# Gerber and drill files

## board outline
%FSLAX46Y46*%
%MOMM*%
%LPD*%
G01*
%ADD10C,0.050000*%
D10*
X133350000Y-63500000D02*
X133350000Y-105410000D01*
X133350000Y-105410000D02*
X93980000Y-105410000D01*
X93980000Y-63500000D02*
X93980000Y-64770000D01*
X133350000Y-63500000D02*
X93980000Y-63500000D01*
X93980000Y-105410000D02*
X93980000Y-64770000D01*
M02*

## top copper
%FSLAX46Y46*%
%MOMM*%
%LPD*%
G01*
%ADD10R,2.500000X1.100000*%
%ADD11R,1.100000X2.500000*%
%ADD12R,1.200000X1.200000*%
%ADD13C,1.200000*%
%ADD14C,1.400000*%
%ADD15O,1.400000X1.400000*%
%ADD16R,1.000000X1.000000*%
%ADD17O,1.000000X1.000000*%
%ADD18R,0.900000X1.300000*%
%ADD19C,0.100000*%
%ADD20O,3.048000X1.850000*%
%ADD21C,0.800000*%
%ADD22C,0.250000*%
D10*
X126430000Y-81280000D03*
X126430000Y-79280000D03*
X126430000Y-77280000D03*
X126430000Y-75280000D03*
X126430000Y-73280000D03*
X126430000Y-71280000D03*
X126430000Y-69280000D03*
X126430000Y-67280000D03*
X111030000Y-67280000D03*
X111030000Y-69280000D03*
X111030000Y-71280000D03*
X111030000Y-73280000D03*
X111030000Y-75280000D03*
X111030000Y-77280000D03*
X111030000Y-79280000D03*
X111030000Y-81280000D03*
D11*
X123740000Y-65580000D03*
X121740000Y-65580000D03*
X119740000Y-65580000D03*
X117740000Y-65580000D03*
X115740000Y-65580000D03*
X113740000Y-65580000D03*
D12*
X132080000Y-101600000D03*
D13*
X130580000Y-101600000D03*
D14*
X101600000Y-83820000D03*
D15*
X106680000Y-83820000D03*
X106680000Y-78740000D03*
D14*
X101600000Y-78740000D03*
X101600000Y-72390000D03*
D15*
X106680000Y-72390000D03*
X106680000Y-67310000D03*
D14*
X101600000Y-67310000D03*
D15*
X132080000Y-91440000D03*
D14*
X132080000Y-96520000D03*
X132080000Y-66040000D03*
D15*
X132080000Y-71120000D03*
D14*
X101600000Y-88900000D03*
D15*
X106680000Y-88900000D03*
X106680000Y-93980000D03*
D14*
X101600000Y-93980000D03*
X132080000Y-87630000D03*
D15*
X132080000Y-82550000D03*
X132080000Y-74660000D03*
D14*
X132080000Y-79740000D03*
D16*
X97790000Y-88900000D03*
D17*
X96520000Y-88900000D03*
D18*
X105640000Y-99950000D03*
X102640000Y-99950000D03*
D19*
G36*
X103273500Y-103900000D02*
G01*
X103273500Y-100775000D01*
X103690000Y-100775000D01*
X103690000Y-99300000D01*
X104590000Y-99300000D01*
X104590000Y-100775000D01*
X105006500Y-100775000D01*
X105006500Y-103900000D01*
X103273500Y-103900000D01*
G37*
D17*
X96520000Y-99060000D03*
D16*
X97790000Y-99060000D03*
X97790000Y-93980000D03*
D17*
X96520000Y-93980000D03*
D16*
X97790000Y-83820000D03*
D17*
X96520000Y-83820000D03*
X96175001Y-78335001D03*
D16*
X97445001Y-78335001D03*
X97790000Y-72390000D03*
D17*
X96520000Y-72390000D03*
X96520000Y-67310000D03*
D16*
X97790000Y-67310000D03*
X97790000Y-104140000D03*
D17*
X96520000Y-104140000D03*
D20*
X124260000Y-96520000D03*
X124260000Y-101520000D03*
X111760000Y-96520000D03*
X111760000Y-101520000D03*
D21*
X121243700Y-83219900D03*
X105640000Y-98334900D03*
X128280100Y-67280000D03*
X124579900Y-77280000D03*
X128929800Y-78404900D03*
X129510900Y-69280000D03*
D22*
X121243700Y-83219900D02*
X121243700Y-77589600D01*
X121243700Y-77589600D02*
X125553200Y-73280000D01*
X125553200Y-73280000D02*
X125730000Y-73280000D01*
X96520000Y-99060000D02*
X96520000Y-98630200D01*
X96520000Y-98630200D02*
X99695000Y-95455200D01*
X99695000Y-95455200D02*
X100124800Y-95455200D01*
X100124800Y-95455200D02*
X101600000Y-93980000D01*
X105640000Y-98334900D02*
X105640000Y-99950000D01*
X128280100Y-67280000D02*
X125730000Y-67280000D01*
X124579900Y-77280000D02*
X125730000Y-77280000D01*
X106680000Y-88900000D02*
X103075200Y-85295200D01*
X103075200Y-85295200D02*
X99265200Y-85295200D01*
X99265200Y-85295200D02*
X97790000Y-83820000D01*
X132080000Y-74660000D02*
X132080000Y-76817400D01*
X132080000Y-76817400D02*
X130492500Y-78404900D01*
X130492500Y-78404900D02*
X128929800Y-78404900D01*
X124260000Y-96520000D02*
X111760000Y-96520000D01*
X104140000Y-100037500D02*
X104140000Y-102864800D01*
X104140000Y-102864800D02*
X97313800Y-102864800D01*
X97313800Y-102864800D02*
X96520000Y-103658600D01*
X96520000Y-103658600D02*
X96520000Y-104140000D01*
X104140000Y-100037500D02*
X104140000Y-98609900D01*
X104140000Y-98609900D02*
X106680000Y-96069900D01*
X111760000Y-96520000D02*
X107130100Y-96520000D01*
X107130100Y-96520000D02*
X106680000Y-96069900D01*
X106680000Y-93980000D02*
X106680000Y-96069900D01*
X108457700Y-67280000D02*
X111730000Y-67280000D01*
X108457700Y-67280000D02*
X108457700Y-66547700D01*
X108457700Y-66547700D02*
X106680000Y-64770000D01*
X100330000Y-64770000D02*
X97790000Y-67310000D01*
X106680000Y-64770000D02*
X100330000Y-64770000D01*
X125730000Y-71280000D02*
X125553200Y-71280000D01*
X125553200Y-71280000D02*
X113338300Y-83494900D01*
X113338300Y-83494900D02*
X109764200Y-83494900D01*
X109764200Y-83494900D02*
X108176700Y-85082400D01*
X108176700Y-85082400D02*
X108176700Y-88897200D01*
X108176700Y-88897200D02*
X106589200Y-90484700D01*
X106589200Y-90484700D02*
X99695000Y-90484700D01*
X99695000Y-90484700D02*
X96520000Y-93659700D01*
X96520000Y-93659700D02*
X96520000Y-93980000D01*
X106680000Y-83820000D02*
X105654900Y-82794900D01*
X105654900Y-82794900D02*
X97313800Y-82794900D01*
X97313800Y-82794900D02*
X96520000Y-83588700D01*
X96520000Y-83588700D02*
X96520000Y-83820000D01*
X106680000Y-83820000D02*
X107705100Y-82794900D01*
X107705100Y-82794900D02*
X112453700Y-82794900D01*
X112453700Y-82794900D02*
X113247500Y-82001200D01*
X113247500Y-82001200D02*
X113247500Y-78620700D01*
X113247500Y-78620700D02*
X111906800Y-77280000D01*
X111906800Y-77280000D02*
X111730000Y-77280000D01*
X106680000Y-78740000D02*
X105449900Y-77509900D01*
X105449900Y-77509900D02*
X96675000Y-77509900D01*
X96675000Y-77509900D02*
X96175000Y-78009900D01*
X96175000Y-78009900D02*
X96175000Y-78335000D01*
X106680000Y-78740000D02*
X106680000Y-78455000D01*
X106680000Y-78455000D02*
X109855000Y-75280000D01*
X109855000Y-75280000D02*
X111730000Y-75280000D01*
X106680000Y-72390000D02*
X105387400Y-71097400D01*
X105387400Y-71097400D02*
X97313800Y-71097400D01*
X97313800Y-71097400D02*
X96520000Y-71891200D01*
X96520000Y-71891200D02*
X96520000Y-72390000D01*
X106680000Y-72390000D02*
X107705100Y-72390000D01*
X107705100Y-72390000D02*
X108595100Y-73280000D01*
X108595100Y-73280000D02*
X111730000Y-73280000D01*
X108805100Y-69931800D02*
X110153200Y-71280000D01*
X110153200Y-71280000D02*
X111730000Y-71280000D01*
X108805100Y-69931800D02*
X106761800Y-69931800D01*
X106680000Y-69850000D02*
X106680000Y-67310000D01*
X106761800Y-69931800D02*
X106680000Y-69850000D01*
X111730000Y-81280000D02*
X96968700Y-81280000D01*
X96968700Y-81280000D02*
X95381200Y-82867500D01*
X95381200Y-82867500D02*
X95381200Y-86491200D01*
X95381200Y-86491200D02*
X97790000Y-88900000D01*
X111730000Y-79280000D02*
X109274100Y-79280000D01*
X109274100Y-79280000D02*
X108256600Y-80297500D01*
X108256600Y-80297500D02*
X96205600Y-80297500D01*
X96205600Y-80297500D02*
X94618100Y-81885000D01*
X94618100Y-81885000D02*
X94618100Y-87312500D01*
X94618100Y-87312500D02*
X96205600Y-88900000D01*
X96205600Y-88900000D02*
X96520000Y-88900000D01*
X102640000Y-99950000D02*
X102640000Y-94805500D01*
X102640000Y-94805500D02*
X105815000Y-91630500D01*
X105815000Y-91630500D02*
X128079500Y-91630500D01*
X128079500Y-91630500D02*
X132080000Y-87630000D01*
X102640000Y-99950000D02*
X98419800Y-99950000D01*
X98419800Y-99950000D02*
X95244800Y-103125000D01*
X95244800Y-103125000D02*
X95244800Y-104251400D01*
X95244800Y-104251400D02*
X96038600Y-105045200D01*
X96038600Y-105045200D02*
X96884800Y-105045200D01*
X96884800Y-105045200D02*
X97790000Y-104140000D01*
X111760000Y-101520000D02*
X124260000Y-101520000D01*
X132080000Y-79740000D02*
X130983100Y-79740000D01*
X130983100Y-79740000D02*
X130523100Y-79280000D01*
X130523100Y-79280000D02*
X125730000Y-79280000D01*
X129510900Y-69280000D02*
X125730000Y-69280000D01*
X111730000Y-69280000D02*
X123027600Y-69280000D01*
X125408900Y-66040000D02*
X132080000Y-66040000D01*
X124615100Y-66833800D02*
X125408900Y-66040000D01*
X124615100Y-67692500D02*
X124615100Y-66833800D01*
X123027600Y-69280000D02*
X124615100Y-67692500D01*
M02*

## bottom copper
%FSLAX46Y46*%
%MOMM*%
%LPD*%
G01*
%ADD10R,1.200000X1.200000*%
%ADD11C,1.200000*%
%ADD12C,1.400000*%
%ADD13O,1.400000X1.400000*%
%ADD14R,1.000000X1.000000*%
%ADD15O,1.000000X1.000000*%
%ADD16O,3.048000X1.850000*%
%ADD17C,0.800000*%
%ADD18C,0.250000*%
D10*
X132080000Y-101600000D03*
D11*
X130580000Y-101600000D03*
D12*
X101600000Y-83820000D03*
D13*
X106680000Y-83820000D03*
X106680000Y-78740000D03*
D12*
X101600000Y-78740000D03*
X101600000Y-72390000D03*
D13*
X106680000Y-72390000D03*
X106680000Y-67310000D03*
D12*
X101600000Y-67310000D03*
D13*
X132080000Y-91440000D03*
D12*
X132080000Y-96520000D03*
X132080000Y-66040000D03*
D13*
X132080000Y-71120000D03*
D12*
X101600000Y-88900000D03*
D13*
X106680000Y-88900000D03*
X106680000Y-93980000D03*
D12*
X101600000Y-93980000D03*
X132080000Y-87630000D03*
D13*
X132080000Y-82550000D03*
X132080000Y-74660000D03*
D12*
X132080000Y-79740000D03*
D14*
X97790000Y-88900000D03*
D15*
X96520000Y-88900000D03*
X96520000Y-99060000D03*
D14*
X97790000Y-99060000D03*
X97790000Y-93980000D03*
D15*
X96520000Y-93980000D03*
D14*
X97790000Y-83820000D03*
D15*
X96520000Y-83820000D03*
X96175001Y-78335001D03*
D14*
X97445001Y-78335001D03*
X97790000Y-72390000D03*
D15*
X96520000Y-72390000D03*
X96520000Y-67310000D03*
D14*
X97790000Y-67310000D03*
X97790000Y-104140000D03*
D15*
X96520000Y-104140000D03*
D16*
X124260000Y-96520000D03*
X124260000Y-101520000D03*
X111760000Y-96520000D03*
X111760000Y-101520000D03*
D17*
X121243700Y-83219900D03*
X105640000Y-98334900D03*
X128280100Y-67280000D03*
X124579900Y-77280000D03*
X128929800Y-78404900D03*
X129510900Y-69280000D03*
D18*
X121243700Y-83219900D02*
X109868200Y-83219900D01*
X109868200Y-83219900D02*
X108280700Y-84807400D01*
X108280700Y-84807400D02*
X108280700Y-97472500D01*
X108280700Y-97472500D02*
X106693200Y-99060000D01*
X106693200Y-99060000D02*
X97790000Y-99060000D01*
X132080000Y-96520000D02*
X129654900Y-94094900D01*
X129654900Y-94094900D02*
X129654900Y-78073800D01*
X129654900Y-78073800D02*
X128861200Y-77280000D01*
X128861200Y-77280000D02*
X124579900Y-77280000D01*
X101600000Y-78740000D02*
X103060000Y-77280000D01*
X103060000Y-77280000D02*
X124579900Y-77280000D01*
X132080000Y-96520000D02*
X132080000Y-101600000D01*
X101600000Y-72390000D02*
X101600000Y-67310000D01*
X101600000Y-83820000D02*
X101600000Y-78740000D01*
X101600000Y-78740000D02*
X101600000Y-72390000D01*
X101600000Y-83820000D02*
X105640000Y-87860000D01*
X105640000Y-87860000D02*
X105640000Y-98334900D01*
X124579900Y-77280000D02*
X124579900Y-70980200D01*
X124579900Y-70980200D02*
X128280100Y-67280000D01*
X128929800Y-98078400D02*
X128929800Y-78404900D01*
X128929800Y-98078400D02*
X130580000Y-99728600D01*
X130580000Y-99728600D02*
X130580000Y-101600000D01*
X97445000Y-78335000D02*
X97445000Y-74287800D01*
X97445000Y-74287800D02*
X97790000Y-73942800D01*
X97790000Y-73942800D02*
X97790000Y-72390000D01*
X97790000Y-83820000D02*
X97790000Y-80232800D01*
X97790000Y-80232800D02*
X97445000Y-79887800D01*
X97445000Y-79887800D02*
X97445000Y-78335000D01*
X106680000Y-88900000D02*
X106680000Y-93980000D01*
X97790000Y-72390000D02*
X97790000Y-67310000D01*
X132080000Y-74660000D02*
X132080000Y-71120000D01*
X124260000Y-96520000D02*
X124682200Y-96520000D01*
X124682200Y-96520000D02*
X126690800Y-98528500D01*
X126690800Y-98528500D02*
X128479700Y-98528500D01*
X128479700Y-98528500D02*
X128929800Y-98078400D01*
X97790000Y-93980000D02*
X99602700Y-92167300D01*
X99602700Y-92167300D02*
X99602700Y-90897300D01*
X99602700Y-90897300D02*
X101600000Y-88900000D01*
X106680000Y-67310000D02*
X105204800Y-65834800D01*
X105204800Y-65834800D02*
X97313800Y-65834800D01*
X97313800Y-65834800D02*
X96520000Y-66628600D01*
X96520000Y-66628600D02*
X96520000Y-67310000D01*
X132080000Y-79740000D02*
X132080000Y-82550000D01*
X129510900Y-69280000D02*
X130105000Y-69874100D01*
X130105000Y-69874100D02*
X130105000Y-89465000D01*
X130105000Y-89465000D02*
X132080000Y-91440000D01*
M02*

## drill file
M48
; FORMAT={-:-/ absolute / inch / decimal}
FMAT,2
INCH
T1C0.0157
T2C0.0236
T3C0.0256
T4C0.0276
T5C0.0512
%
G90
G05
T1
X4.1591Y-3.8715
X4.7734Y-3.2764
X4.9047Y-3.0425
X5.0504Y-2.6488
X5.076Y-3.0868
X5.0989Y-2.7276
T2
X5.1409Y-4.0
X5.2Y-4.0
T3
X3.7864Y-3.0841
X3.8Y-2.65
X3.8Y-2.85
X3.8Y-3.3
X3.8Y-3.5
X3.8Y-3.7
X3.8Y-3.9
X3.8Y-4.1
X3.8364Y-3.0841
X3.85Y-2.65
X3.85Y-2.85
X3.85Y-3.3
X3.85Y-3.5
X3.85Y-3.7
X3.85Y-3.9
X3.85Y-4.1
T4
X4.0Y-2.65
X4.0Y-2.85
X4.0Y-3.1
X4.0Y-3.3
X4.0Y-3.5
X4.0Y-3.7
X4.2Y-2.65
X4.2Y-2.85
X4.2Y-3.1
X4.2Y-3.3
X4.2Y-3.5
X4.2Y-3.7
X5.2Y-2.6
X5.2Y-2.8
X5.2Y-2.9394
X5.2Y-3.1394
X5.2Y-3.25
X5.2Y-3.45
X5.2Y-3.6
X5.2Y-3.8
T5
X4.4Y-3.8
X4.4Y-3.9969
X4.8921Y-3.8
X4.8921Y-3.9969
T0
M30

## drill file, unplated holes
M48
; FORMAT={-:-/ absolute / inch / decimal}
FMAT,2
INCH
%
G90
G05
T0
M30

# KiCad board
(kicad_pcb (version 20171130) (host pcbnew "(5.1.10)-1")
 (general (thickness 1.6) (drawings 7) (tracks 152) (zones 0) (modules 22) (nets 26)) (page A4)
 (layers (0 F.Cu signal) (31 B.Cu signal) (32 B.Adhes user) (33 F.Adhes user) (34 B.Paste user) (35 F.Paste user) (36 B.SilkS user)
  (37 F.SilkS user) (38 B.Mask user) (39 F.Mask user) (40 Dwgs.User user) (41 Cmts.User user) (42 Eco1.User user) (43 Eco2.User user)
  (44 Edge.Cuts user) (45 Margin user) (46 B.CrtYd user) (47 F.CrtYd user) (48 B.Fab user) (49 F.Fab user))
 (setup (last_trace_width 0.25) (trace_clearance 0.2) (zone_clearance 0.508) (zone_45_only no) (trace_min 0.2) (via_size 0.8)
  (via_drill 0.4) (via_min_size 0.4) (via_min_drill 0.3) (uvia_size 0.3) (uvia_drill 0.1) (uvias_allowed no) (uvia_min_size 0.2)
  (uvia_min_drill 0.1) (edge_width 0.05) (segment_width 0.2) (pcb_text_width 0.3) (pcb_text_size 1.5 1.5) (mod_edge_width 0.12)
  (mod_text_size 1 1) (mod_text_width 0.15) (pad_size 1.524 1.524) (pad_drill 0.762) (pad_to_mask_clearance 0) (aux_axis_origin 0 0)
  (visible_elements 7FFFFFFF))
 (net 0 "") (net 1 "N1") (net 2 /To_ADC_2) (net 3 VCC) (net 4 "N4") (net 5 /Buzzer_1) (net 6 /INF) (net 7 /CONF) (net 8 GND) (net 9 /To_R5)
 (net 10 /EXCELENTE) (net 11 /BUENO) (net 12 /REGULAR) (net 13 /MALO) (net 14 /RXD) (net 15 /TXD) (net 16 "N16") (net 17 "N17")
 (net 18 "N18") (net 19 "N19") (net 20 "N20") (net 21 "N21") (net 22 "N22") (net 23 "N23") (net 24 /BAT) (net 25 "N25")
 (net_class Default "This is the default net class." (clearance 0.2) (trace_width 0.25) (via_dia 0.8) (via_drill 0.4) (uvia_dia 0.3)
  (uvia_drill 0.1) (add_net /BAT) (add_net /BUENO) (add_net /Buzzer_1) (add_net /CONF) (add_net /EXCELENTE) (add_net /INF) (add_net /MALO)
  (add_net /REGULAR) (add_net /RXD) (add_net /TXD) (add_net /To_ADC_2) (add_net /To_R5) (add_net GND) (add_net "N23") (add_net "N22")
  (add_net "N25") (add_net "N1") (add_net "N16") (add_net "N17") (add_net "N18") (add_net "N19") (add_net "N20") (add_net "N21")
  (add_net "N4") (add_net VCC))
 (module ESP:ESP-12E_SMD (layer F.Cu) (at 125.73 81.28 180)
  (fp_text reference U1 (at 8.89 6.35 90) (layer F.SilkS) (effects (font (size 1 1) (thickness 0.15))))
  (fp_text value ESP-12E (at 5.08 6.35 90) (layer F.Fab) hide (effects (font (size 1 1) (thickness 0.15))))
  (pad 1 smd rect (at 0 0 180) (size 2.5 1.1) (drill (offset -0.7 0)) (layers F.Cu F.Paste F.Mask) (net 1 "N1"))
  (pad 2 smd rect (at 0 2 180) (size 2.5 1.1) (drill (offset -0.7 0)) (layers F.Cu F.Paste F.Mask) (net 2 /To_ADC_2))
  (pad 3 smd rect (at 0 4 180) (size 2.5 1.1) (drill (offset -0.7 0)) (layers F.Cu F.Paste F.Mask) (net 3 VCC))
  (pad 4 smd rect (at 0 6 180) (size 2.5 1.1) (drill (offset -0.7 0)) (layers F.Cu F.Paste F.Mask) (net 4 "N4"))
  (pad 5 smd rect (at 0 8 180) (size 2.5 1.1) (drill (offset -0.7 0)) (layers F.Cu F.Paste F.Mask) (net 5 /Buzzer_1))
  (pad 6 smd rect (at 0 10 180) (size 2.5 1.1) (drill (offset -0.7 0)) (layers F.Cu F.Paste F.Mask) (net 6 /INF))
  (pad 7 smd rect (at 0 12 180) (size 2.5 1.1) (drill (offset -0.7 0)) (layers F.Cu F.Paste F.Mask) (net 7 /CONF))
  (pad 8 smd rect (at 0 14 180) (size 2.5 1.1) (drill (offset -0.7 0)) (layers F.Cu F.Paste F.Mask) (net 3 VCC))
  (pad 9 smd rect (at 14 14 180) (size 2.5 1.1) (drill (offset 0.7 0)) (layers F.Cu F.Paste F.Mask) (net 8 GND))
  (pad 10 smd rect (at 14 12 180) (size 2.5 1.1) (drill (offset 0.7 0)) (layers F.Cu F.Paste F.Mask) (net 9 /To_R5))
  (pad 11 smd rect (at 14 10 180) (size 2.5 1.1) (drill (offset 0.7 0)) (layers F.Cu F.Paste F.Mask) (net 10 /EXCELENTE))
  (pad 12 smd rect (at 14 8 180) (size 2.5 1.1) (drill (offset 0.7 0)) (layers F.Cu F.Paste F.Mask) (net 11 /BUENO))
  (pad 13 smd rect (at 14 6 180) (size 2.5 1.1) (drill (offset 0.7 0)) (layers F.Cu F.Paste F.Mask) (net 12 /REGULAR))
  (pad 14 smd rect (at 14 4 180) (size 2.5 1.1) (drill (offset 0.7 0)) (layers F.Cu F.Paste F.Mask) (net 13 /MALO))
  (pad 15 smd rect (at 14 2 180) (size 2.5 1.1) (drill (offset 0.7 0)) (layers F.Cu F.Paste F.Mask) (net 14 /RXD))
  (pad 16 smd rect (at 14 0 180) (size 2.5 1.1) (drill (offset 0.7 0)) (layers F.Cu F.Paste F.Mask) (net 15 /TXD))
  (pad 17 smd rect (at 1.99 15 270) (size 2.5 1.1) (drill (offset -0.7 0)) (layers F.Cu F.Paste F.Mask) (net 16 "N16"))
  (pad 18 smd rect (at 3.99 15 270) (size 2.5 1.1) (drill (offset -0.7 0)) (layers F.Cu F.Paste F.Mask) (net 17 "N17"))
  (pad 19 smd rect (at 5.99 15 270) (size 2.5 1.1) (drill (offset -0.7 0)) (layers F.Cu F.Paste F.Mask) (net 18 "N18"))
  (pad 20 smd rect (at 7.99 15 270) (size 2.5 1.1) (drill (offset -0.7 0)) (layers F.Cu F.Paste F.Mask) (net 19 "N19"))
  (pad 21 smd rect (at 9.99 15 270) (size 2.5 1.1) (drill (offset -0.7 0)) (layers F.Cu F.Paste F.Mask) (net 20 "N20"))
  (pad 22 smd rect (at 11.99 15 270) (size 2.5 1.1) (drill (offset -0.7 0)) (layers F.Cu F.Paste F.Mask) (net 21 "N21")))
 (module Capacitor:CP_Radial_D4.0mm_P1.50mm (layer F.Cu) (at 132.08 101.6 180)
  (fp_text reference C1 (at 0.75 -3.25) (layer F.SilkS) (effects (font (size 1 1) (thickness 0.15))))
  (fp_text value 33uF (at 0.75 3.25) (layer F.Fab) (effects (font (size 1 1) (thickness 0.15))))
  (pad 1 thru_hole rect (at 0 0 180) (size 1.2 1.2) (drill 0.6) (layers *.Cu *.Mask) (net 3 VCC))
  (pad 2 thru_hole circle (at 1.5 0 180) (size 1.2 1.2) (drill 0.6) (layers *.Cu *.Mask) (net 8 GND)))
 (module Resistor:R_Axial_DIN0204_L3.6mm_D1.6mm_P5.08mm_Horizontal (layer F.Cu) (at 101.6 83.82)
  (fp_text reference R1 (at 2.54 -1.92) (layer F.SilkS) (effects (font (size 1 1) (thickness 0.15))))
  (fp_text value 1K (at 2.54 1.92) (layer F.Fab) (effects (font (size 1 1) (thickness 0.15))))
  (pad 1 thru_hole circle (at 0 0) (size 1.4 1.4) (drill 0.7) (layers *.Cu *.Mask) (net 3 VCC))
  (pad 2 thru_hole oval (at 5.08 0) (size 1.4 1.4) (drill 0.7) (layers *.Cu *.Mask) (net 13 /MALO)))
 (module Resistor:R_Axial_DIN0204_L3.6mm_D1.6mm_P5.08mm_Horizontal (layer F.Cu) (at 101.6 78.74)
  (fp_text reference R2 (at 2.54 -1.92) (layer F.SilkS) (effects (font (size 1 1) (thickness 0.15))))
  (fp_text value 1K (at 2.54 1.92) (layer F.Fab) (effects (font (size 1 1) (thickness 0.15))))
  (pad 2 thru_hole oval (at 5.08 0) (size 1.4 1.4) (drill 0.7) (layers *.Cu *.Mask) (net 12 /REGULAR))
  (pad 1 thru_hole circle (at 0 0) (size 1.4 1.4) (drill 0.7) (layers *.Cu *.Mask) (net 3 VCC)))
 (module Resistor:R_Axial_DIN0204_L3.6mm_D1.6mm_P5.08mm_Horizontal (layer F.Cu) (at 101.6 72.39)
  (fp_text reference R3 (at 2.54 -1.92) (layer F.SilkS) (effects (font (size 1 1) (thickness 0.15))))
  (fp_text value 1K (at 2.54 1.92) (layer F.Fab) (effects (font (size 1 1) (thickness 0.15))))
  (pad 1 thru_hole circle (at 0 0) (size 1.4 1.4) (drill 0.7) (layers *.Cu *.Mask) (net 3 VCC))
  (pad 2 thru_hole oval (at 5.08 0) (size 1.4 1.4) (drill 0.7) (layers *.Cu *.Mask) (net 11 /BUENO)))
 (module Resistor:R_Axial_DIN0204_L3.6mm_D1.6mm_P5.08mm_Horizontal (layer F.Cu) (at 101.6 67.31)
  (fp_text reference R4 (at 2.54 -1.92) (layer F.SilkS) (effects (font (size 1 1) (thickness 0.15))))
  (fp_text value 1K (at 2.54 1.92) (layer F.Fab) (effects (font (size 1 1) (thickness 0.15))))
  (pad 2 thru_hole oval (at 5.08 0) (size 1.4 1.4) (drill 0.7) (layers *.Cu *.Mask) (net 10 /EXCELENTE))
  (pad 1 thru_hole circle (at 0 0) (size 1.4 1.4) (drill 0.7) (layers *.Cu *.Mask) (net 3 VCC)))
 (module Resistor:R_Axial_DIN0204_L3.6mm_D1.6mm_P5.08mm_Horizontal (layer F.Cu) (at 132.08 96.52 90)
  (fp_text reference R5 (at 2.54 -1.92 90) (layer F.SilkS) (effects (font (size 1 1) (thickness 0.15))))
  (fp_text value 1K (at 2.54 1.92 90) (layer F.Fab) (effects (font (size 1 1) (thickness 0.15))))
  (pad 2 thru_hole oval (at 5.08 0 90) (size 1.4 1.4) (drill 0.7) (layers *.Cu *.Mask) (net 7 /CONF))
  (pad 1 thru_hole circle (at 0 0 90) (size 1.4 1.4) (drill 0.7) (layers *.Cu *.Mask) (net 3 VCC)))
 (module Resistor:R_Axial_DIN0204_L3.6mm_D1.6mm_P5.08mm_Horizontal (layer F.Cu) (at 132.08 66.04 270)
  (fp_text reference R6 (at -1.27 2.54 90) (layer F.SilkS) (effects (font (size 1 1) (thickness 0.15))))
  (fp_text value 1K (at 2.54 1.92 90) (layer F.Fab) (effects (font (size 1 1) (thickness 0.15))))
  (pad 1 thru_hole circle (at 0 0 270) (size 1.4 1.4) (drill 0.7) (layers *.Cu *.Mask) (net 9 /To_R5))
  (pad 2 thru_hole oval (at 5.08 0 270) (size 1.4 1.4) (drill 0.7) (layers *.Cu *.Mask) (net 8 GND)))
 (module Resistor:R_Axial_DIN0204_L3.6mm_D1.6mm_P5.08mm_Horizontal (layer F.Cu) (at 101.6 88.9)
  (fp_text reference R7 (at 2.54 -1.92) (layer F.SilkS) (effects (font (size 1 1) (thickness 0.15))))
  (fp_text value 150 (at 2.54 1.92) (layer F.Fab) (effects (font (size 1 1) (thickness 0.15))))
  (pad 1 thru_hole circle (at 0 0) (size 1.4 1.4) (drill 0.7) (layers *.Cu *.Mask) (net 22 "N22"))
  (pad 2 thru_hole oval (at 5.08 0) (size 1.4 1.4) (drill 0.7) (layers *.Cu *.Mask) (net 8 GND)))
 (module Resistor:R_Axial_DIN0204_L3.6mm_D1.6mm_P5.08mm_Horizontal (layer F.Cu) (at 101.6 93.98)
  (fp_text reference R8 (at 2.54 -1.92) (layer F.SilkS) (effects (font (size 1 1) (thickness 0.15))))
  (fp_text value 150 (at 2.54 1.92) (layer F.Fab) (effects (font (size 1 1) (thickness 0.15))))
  (pad 2 thru_hole oval (at 5.08 0) (size 1.4 1.4) (drill 0.7) (layers *.Cu *.Mask) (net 8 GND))
  (pad 1 thru_hole circle (at 0 0) (size 1.4 1.4) (drill 0.7) (layers *.Cu *.Mask) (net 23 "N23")))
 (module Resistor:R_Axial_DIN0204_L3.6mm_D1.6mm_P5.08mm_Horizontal (layer F.Cu) (at 132.08 87.63 90)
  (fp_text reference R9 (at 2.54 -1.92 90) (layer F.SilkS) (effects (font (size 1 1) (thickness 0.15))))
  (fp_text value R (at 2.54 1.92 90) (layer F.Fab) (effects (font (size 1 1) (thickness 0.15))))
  (pad 1 thru_hole circle (at 0 0 90) (size 1.4 1.4) (drill 0.7) (layers *.Cu *.Mask) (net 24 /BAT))
  (pad 2 thru_hole oval (at 5.08 0 90) (size 1.4 1.4) (drill 0.7) (layers *.Cu *.Mask) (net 2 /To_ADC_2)))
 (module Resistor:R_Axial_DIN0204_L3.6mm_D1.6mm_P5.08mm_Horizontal (layer F.Cu) (at 132.08 79.74 90)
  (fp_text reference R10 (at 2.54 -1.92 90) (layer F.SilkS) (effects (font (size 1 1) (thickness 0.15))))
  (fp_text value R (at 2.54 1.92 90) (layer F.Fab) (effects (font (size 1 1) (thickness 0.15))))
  (pad 2 thru_hole oval (at 5.08 0 90) (size 1.4 1.4) (drill 0.7) (layers *.Cu *.Mask) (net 8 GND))
  (pad 1 thru_hole circle (at 0 0 90) (size 1.4 1.4) (drill 0.7) (layers *.Cu *.Mask) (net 2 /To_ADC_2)))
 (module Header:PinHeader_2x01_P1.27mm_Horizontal (layer F.Cu) (at 97.79 88.9 180)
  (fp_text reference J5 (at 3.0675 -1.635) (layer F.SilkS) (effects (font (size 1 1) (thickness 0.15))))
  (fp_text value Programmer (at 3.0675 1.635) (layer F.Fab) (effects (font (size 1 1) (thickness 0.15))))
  (pad 1 thru_hole rect (at 0 0 180) (size 1 1) (drill 0.65) (layers *.Cu *.Mask) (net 15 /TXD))
  (pad 2 thru_hole oval (at 1.27 0 180) (size 1 1) (drill 0.65) (layers *.Cu *.Mask) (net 14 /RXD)))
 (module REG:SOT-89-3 (layer F.Cu) (at 104.14 101.6 270)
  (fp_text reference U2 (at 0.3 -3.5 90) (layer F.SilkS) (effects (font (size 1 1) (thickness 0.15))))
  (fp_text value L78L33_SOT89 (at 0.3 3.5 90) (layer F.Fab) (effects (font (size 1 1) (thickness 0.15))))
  (pad 1 smd rect (at -1.65 -1.5 270) (size 1.3 0.9) (layers F.Cu F.Paste F.Mask) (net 3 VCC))
  (pad 3 smd rect (at -1.65 1.5 270) (size 1.3 0.9) (layers F.Cu F.Paste F.Mask) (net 24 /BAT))
  (pad 2 smd custom (at -1.5625 0 270) (size 1.475 0.9) (layers F.Cu F.Paste F.Mask) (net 8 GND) (zone_connect 2)
   (options (clearance outline) (anchor rect)) (primitives)))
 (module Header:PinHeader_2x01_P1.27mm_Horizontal (layer F.Cu) (at 97.79 99.06 180)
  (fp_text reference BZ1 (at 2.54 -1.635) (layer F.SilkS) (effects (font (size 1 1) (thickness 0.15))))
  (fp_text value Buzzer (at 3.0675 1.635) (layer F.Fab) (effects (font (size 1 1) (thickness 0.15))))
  (pad 2 thru_hole oval (at 1.27 0 180) (size 1 1) (drill 0.65) (layers *.Cu *.Mask) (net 23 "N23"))
  (pad 1 thru_hole rect (at 0 0 180) (size 1 1) (drill 0.65) (layers *.Cu *.Mask) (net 5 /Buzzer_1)))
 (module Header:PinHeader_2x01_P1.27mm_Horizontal (layer F.Cu) (at 97.79 93.98 180)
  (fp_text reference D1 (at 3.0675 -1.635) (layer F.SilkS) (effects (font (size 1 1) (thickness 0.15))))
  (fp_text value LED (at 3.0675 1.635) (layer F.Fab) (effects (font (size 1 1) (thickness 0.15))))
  (pad 1 thru_hole rect (at 0 0 180) (size 1 1) (drill 0.65) (layers *.Cu *.Mask) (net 22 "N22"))
  (pad 2 thru_hole oval (at 1.27 0 180) (size 1 1) (drill 0.65) (layers *.Cu *.Mask) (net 6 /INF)))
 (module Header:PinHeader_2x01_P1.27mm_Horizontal (layer F.Cu) (at 97.79 83.82 180)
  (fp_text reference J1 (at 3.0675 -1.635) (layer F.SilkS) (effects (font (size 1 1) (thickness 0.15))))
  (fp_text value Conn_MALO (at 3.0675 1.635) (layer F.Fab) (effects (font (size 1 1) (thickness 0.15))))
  (pad 1 thru_hole rect (at 0 0 180) (size 1 1) (drill 0.65) (layers *.Cu *.Mask) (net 8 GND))
  (pad 2 thru_hole oval (at 1.27 0 180) (size 1 1) (drill 0.65) (layers *.Cu *.Mask) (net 13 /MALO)))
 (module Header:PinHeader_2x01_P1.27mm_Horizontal (layer F.Cu) (at 97.445001 78.335001 180)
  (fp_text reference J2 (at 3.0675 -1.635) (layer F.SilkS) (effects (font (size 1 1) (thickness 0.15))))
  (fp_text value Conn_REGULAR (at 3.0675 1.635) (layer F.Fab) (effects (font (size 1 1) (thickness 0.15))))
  (pad 2 thru_hole oval (at 1.27 0 180) (size 1 1) (drill 0.65) (layers *.Cu *.Mask) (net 12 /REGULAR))
  (pad 1 thru_hole rect (at 0 0 180) (size 1 1) (drill 0.65) (layers *.Cu *.Mask) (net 8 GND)))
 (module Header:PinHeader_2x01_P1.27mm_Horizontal (layer F.Cu) (at 97.79 72.39 180)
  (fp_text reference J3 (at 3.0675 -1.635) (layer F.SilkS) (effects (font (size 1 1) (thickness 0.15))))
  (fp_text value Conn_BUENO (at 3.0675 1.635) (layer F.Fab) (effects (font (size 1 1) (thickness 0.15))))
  (pad 1 thru_hole rect (at 0 0 180) (size 1 1) (drill 0.65) (layers *.Cu *.Mask) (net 8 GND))
  (pad 2 thru_hole oval (at 1.27 0 180) (size 1 1) (drill 0.65) (layers *.Cu *.Mask) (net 11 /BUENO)))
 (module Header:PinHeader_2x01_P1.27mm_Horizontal (layer F.Cu) (at 97.79 67.31 180)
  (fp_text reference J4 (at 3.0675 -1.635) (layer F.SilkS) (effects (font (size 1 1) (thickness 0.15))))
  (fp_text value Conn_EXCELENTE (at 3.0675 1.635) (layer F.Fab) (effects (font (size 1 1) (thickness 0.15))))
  (pad 2 thru_hole oval (at 1.27 0 180) (size 1 1) (drill 0.65) (layers *.Cu *.Mask) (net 10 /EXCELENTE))
  (pad 1 thru_hole rect (at 0 0 180) (size 1 1) (drill 0.65) (layers *.Cu *.Mask) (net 8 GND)))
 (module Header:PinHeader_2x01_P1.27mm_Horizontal (layer F.Cu) (at 97.79 104.14 180)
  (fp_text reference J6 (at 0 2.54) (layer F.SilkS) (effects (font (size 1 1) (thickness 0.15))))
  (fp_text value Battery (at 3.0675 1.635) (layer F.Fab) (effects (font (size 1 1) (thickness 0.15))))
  (pad 1 thru_hole rect (at 0 0 180) (size 1 1) (drill 0.65) (layers *.Cu *.Mask) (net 24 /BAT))
  (pad 2 thru_hole oval (at 1.27 0 180) (size 1 1) (drill 0.65) (layers *.Cu *.Mask) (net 8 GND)))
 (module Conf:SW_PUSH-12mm (layer F.Cu) (at 111.76 96.52)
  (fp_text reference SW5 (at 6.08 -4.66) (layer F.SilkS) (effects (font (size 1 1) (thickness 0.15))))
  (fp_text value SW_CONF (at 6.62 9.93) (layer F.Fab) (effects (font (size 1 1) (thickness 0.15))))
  (pad 1 thru_hole oval (at 12.5 0) (size 3.048 1.85) (drill 1.3) (layers *.Cu *.Mask) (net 8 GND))
  (pad 2 thru_hole oval (at 12.5 5) (size 3.048 1.85) (drill 1.3) (layers *.Cu *.Mask) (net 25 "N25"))
  (pad 1 thru_hole oval (at 0 0) (size 3.048 1.85) (drill 1.3) (layers *.Cu *.Mask) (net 8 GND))
  (pad 2 thru_hole oval (at 0 5) (size 3.048 1.85) (drill 1.3) (layers *.Cu *.Mask) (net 25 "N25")))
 (gr_line (start 133.35 63.5) (end 133.35 105.41) (layer Edge.Cuts) (width 0.05))
 (gr_line (start 133.35 105.41) (end 93.98 105.41) (layer Edge.Cuts) (width 0.05))
 (gr_line (start 93.98 63.5) (end 93.98 64.77) (layer Edge.Cuts) (width 0.05))
 (gr_line (start 133.35 63.5) (end 93.98 63.5) (layer Edge.Cuts) (width 0.05))
 (gr_line (start 93.98 105.41) (end 93.98 64.77) (layer Edge.Cuts) (width 0.05))
 (segment (start 121.2437 83.2199) (end 121.2437 77.5896) (width 0.25) (layer F.Cu) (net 5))
 (segment (start 121.2437 77.5896) (end 125.5532 73.28) (width 0.25) (layer F.Cu) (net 5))
 (segment (start 125.5532 73.28) (end 125.73 73.28) (width 0.25) (layer F.Cu) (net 5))
 (segment (start 121.2437 83.2199) (end 109.8682 83.2199) (width 0.25) (layer B.Cu) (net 5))
 (segment (start 109.8682 83.2199) (end 108.2807 84.8074) (width 0.25) (layer B.Cu) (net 5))
 (segment (start 108.2807 84.8074) (end 108.2807 97.4725) (width 0.25) (layer B.Cu) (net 5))
 (segment (start 108.2807 97.4725) (end 106.6932 99.06) (width 0.25) (layer B.Cu) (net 5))
 (segment (start 106.6932 99.06) (end 97.79 99.06) (width 0.25) (layer B.Cu) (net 5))
 (via (at 121.2437 83.2199) (size 0.8) (layers F.Cu B.Cu) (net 5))
 (segment (start 96.52 99.06) (end 96.52 98.6302) (width 0.25) (layer F.Cu) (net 23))
 (segment (start 96.52 98.6302) (end 99.695 95.4552) (width 0.25) (layer F.Cu) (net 23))
 (segment (start 99.695 95.4552) (end 100.1248 95.4552) (width 0.25) (layer F.Cu) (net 23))
 (segment (start 100.1248 95.4552) (end 101.6 93.98) (width 0.25) (layer F.Cu) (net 23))
 (segment (start 132.08 96.52) (end 129.6549 94.0949) (width 0.25) (layer B.Cu) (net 3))
 (segment (start 129.6549 94.0949) (end 129.6549 78.0738) (width 0.25) (layer B.Cu) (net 3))
 (segment (start 129.6549 78.0738) (end 128.8612 77.28) (width 0.25) (layer B.Cu) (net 3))
 (segment (start 128.8612 77.28) (end 124.5799 77.28) (width 0.25) (layer B.Cu) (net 3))
 (segment (start 101.6 78.74) (end 103.06 77.28) (width 0.25) (layer B.Cu) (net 3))
 (segment (start 103.06 77.28) (end 124.5799 77.28) (width 0.25) (layer B.Cu) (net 3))
 (segment (start 132.08 96.52) (end 132.08 101.6) (width 0.25) (layer B.Cu) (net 3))
 (segment (start 101.6 72.39) (end 101.6 67.31) (width 0.25) (layer B.Cu) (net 3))
 (segment (start 101.6 83.82) (end 101.6 78.74) (width 0.25) (layer B.Cu) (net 3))
 (segment (start 101.6 78.74) (end 101.6 72.39) (width 0.25) (layer B.Cu) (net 3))
 (segment (start 105.64 98.3349) (end 105.64 99.95) (width 0.25) (layer F.Cu) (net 3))
 (segment (start 101.6 83.82) (end 105.64 87.86) (width 0.25) (layer B.Cu) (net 3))
 (segment (start 105.64 87.86) (end 105.64 98.3349) (width 0.25) (layer B.Cu) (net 3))
 (segment (start 128.2801 67.28) (end 125.73 67.28) (width 0.25) (layer F.Cu) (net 3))
 (segment (start 124.5799 77.28) (end 124.5799 70.9802) (width 0.25) (layer B.Cu) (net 3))
 (segment (start 124.5799 70.9802) (end 128.2801 67.28) (width 0.25) (layer B.Cu) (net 3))
 (segment (start 124.5799 77.28) (end 125.73 77.28) (width 0.25) (layer F.Cu) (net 3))
 (via (at 105.64 98.3349) (size 0.8) (layers F.Cu B.Cu) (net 3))
 (via (at 128.2801 67.28) (size 0.8) (layers F.Cu B.Cu) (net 3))
 (via (at 124.5799 77.28) (size 0.8) (layers F.Cu B.Cu) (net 3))
 (segment (start 106.68 88.9) (end 103.0752 85.2952) (width 0.25) (layer F.Cu) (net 8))
 (segment (start 103.0752 85.2952) (end 99.2652 85.2952) (width 0.25) (layer F.Cu) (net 8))
 (segment (start 99.2652 85.2952) (end 97.79 83.82) (width 0.25) (layer F.Cu) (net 8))
 (segment (start 132.08 74.66) (end 132.08 76.8174) (width 0.25) (layer F.Cu) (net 8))
 (segment (start 132.08 76.8174) (end 130.4925 78.4049) (width 0.25) (layer F.Cu) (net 8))
 (segment (start 130.4925 78.4049) (end 128.9298 78.4049) (width 0.25) (layer F.Cu) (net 8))
 (segment (start 128.9298 98.0784) (end 128.9298 78.4049) (width 0.25) (layer B.Cu) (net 8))
 (segment (start 128.9298 98.0784) (end 130.58 99.7286) (width 0.25) (layer B.Cu) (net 8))
 (segment (start 130.58 99.7286) (end 130.58 101.6) (width 0.25) (layer B.Cu) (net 8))
 (segment (start 124.26 96.52) (end 111.76 96.52) (width 0.25) (layer F.Cu) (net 8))
 (segment (start 104.14 100.0375) (end 104.14 102.8648) (width 0.25) (layer F.Cu) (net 8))
 (segment (start 104.14 102.8648) (end 97.3138 102.8648) (width 0.25) (layer F.Cu) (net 8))
 (segment (start 97.3138 102.8648) (end 96.52 103.6586) (width 0.25) (layer F.Cu) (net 8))
 (segment (start 96.52 103.6586) (end 96.52 104.14) (width 0.25) (layer F.Cu) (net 8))
 (segment (start 97.445 78.335) (end 97.445 74.2878) (width 0.25) (layer B.Cu) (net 8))
 (segment (start 97.445 74.2878) (end 97.79 73.9428) (width 0.25) (layer B.Cu) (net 8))
 (segment (start 97.79 73.9428) (end 97.79 72.39) (width 0.25) (layer B.Cu) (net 8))
 (segment (start 104.14 100.0375) (end 104.14 98.6099) (width 0.25) (layer F.Cu) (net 8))
 (segment (start 104.14 98.6099) (end 106.68 96.0699) (width 0.25) (layer F.Cu) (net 8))
 (segment (start 97.79 83.82) (end 97.79 80.2328) (width 0.25) (layer B.Cu) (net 8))
 (segment (start 97.79 80.2328) (end 97.445 79.8878) (width 0.25) (layer B.Cu) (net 8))
 (segment (start 97.445 79.8878) (end 97.445 78.335) (width 0.25) (layer B.Cu) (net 8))
 (segment (start 111.76 96.52) (end 107.1301 96.52) (width 0.25) (layer F.Cu) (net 8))
 (segment (start 107.1301 96.52) (end 106.68 96.0699) (width 0.25) (layer F.Cu) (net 8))
 (segment (start 106.68 88.9) (end 106.68 93.98) (width 0.25) (layer B.Cu) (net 8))
 (segment (start 97.79 72.39) (end 97.79 67.31) (width 0.25) (layer B.Cu) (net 8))
 (segment (start 132.08 74.66) (end 132.08 71.12) (width 0.25) (layer B.Cu) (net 8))
 (segment (start 124.26 96.52) (end 124.6822 96.52) (width 0.25) (layer B.Cu) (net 8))
 (segment (start 124.6822 96.52) (end 126.6908 98.5285) (width 0.25) (layer B.Cu) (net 8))
 (segment (start 126.6908 98.5285) (end 128.4797 98.5285) (width 0.25) (layer B.Cu) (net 8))
 (segment (start 128.4797 98.5285) (end 128.9298 98.0784) (width 0.25) (layer B.Cu) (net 8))
 (segment (start 106.68 93.98) (end 106.68 96.0699) (width 0.25) (layer F.Cu) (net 8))
 (segment (start 108.4577 67.28) (end 111.73 67.28) (width 0.25) (layer F.Cu) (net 8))
 (via (at 128.9298 78.4049) (size 0.8) (layers F.Cu B.Cu) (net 8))
 (segment (start 108.4577 67.28) (end 108.4577 66.5477) (width 0.25) (layer F.Cu) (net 8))
 (segment (start 108.4577 66.5477) (end 106.68 64.77) (width 0.25) (layer F.Cu) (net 8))
 (segment (start 100.33 64.77) (end 97.79 67.31) (width 0.25) (layer F.Cu) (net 8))
 (segment (start 106.68 64.77) (end 100.33 64.77) (width 0.25) (layer F.Cu) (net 8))
 (segment (start 97.79 93.98) (end 99.6027 92.1673) (width 0.25) (layer B.Cu) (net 22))
 (segment (start 99.6027 92.1673) (end 99.6027 90.8973) (width 0.25) (layer B.Cu) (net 22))
 (segment (start 99.6027 90.8973) (end 101.6 88.9) (width 0.25) (layer B.Cu) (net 22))
 (segment (start 125.73 71.28) (end 125.5532 71.28) (width 0.25) (layer F.Cu) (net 6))
 (segment (start 125.5532 71.28) (end 113.3383 83.4949) (width 0.25) (layer F.Cu) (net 6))
 (segment (start 113.3383 83.4949) (end 109.7642 83.4949) (width 0.25) (layer F.Cu) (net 6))
 (segment (start 109.7642 83.4949) (end 108.1767 85.0824) (width 0.25) (layer F.Cu) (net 6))
 (segment (start 108.1767 85.0824) (end 108.1767 88.8972) (width 0.25) (layer F.Cu) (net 6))
 (segment (start 108.1767 88.8972) (end 106.5892 90.4847) (width 0.25) (layer F.Cu) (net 6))
 (segment (start 106.5892 90.4847) (end 99.695 90.4847) (width 0.25) (layer F.Cu) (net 6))
 (segment (start 99.695 90.4847) (end 96.52 93.6597) (width 0.25) (layer F.Cu) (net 6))
 (segment (start 96.52 93.6597) (end 96.52 93.98) (width 0.25) (layer F.Cu) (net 6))
 (segment (start 106.68 83.82) (end 105.6549 82.7949) (width 0.25) (layer F.Cu) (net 13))
 (segment (start 105.6549 82.7949) (end 97.3138 82.7949) (width 0.25) (layer F.Cu) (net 13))
 (segment (start 97.3138 82.7949) (end 96.52 83.5887) (width 0.25) (layer F.Cu) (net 13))
 (segment (start 96.52 83.5887) (end 96.52 83.82) (width 0.25) (layer F.Cu) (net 13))
 (segment (start 106.68 83.82) (end 107.7051 82.7949) (width 0.25) (layer F.Cu) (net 13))
 (segment (start 107.7051 82.7949) (end 112.4537 82.7949) (width 0.25) (layer F.Cu) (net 13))
 (segment (start 112.4537 82.7949) (end 113.2475 82.0012) (width 0.25) (layer F.Cu) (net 13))
 (segment (start 113.2475 82.0012) (end 113.2475 78.6207) (width 0.25) (layer F.Cu) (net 13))
 (segment (start 113.2475 78.6207) (end 111.9068 77.28) (width 0.25) (layer F.Cu) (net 13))
 (segment (start 111.9068 77.28) (end 111.73 77.28) (width 0.25) (layer F.Cu) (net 13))
 (segment (start 106.68 78.74) (end 105.4499 77.5099) (width 0.25) (layer F.Cu) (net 12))
 (segment (start 105.4499 77.5099) (end 96.675 77.5099) (width 0.25) (layer F.Cu) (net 12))
 (segment (start 96.675 77.5099) (end 96.175 78.0099) (width 0.25) (layer F.Cu) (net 12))
 (segment (start 96.175 78.0099) (end 96.175 78.335) (width 0.25) (layer F.Cu) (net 12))
 (segment (start 106.68 78.74) (end 106.68 78.455) (width 0.25) (layer F.Cu) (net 12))
 (segment (start 106.68 78.455) (end 109.855 75.28) (width 0.25) (layer F.Cu) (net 12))
 (segment (start 109.855 75.28) (end 111.73 75.28) (width 0.25) (layer F.Cu) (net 12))
 (segment (start 106.68 72.39) (end 105.3874 71.0974) (width 0.25) (layer F.Cu) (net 11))
 (segment (start 105.3874 71.0974) (end 97.3138 71.0974) (width 0.25) (layer F.Cu) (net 11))
 (segment (start 97.3138 71.0974) (end 96.52 71.8912) (width 0.25) (layer F.Cu) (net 11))
 (segment (start 96.52 71.8912) (end 96.52 72.39) (width 0.25) (layer F.Cu) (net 11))
 (segment (start 106.68 72.39) (end 107.7051 72.39) (width 0.25) (layer F.Cu) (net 11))
 (segment (start 107.7051 72.39) (end 108.5951 73.28) (width 0.25) (layer F.Cu) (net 11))
 (segment (start 108.5951 73.28) (end 111.73 73.28) (width 0.25) (layer F.Cu) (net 11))
 (segment (start 106.68 67.31) (end 105.2048 65.8348) (width 0.25) (layer B.Cu) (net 10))
 (segment (start 105.2048 65.8348) (end 97.3138 65.8348) (width 0.25) (layer B.Cu) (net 10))
 (segment (start 97.3138 65.8348) (end 96.52 66.6286) (width 0.25) (layer B.Cu) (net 10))
 (segment (start 96.52 66.6286) (end 96.52 67.31) (width 0.25) (layer B.Cu) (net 10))
 (segment (start 108.8051 69.9318) (end 110.1532 71.28) (width 0.25) (layer F.Cu) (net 10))
 (segment (start 110.1532 71.28) (end 111.73 71.28) (width 0.25) (layer F.Cu) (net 10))
 (segment (start 108.8051 69.9318) (end 106.7618 69.9318) (width 0.25) (layer F.Cu) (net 10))
 (segment (start 106.68 69.85) (end 106.68 67.31) (width 0.25) (layer F.Cu) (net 10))
 (segment (start 106.7618 69.9318) (end 106.68 69.85) (width 0.25) (layer F.Cu) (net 10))
 (segment (start 111.73 81.28) (end 96.9687 81.28) (width 0.25) (layer F.Cu) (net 15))
 (segment (start 96.9687 81.28) (end 95.3812 82.8675) (width 0.25) (layer F.Cu) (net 15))
 (segment (start 95.3812 82.8675) (end 95.3812 86.4912) (width 0.25) (layer F.Cu) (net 15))
 (segment (start 95.3812 86.4912) (end 97.79 88.9) (width 0.25) (layer F.Cu) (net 15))
 (segment (start 111.73 79.28) (end 109.2741 79.28) (width 0.25) (layer F.Cu) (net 14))
 (segment (start 109.2741 79.28) (end 108.2566 80.2975) (width 0.25) (layer F.Cu) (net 14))
 (segment (start 108.2566 80.2975) (end 96.2056 80.2975) (width 0.25) (layer F.Cu) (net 14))
 (segment (start 96.2056 80.2975) (end 94.6181 81.885) (width 0.25) (layer F.Cu) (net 14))
 (segment (start 94.6181 81.885) (end 94.6181 87.3125) (width 0.25) (layer F.Cu) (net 14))
 (segment (start 94.6181 87.3125) (end 96.2056 88.9) (width 0.25) (layer F.Cu) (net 14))
 (segment (start 96.2056 88.9) (end 96.52 88.9) (width 0.25) (layer F.Cu) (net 14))
 (segment (start 102.64 99.95) (end 102.64 94.8055) (width 0.25) (layer F.Cu) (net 24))
 (segment (start 102.64 94.8055) (end 105.815 91.6305) (width 0.25) (layer F.Cu) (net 24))
 (segment (start 105.815 91.6305) (end 128.0795 91.6305) (width 0.25) (layer F.Cu) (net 24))
 (segment (start 128.0795 91.6305) (end 132.08 87.63) (width 0.25) (layer F.Cu) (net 24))
 (segment (start 102.64 99.95) (end 98.4198 99.95) (width 0.25) (layer F.Cu) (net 24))
 (segment (start 98.4198 99.95) (end 95.2448 103.125) (width 0.25) (layer F.Cu) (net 24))
 (segment (start 95.2448 103.125) (end 95.2448 104.2514) (width 0.25) (layer F.Cu) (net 24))
 (segment (start 95.2448 104.2514) (end 96.0386 105.0452) (width 0.25) (layer F.Cu) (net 24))
 (segment (start 96.0386 105.0452) (end 96.8848 105.0452) (width 0.25) (layer F.Cu) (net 24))
 (segment (start 96.8848 105.0452) (end 97.79 104.14) (width 0.25) (layer F.Cu) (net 24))
 (segment (start 111.76 101.52) (end 124.26 101.52) (width 0.25) (layer F.Cu) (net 25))
 (segment (start 132.08 79.74) (end 132.08 82.55) (width 0.25) (layer B.Cu) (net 2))
 (segment (start 132.08 79.74) (end 130.9831 79.74) (width 0.25) (layer F.Cu) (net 2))
 (segment (start 130.9831 79.74) (end 130.5231 79.28) (width 0.25) (layer F.Cu) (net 2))
 (segment (start 130.5231 79.28) (end 125.73 79.28) (width 0.25) (layer F.Cu) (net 2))
 (segment (start 129.5109 69.28) (end 125.73 69.28) (width 0.25) (layer F.Cu) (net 7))
 (segment (start 129.5109 69.28) (end 130.105 69.8741) (width 0.25) (layer B.Cu) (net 7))
 (segment (start 130.105 69.8741) (end 130.105 89.465) (width 0.25) (layer B.Cu) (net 7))
 (segment (start 130.105 89.465) (end 132.08 91.44) (width 0.25) (layer B.Cu) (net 7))
 (via (at 129.5109 69.28) (size 0.8) (layers F.Cu B.Cu) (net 7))
 (segment (start 111.73 69.28) (end 123.0276 69.28) (width 0.25) (layer F.Cu) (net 9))
 (segment (start 125.4089 66.04) (end 132.08 66.04) (width 0.25) (layer F.Cu) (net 9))
 (segment (start 124.6151 66.8338) (end 125.4089 66.04) (width 0.25) (layer F.Cu) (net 9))
 (segment (start 124.6151 67.6925) (end 124.6151 66.8338) (width 0.25) (layer F.Cu) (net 9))
 (segment (start 123.0276 69.28) (end 124.6151 67.6925) (width 0.25) (layer F.Cu) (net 9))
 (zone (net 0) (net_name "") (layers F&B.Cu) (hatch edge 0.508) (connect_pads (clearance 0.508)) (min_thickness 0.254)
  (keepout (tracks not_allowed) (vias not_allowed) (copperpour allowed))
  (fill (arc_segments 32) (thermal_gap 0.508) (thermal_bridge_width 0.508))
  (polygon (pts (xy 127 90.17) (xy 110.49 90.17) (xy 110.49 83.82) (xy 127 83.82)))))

